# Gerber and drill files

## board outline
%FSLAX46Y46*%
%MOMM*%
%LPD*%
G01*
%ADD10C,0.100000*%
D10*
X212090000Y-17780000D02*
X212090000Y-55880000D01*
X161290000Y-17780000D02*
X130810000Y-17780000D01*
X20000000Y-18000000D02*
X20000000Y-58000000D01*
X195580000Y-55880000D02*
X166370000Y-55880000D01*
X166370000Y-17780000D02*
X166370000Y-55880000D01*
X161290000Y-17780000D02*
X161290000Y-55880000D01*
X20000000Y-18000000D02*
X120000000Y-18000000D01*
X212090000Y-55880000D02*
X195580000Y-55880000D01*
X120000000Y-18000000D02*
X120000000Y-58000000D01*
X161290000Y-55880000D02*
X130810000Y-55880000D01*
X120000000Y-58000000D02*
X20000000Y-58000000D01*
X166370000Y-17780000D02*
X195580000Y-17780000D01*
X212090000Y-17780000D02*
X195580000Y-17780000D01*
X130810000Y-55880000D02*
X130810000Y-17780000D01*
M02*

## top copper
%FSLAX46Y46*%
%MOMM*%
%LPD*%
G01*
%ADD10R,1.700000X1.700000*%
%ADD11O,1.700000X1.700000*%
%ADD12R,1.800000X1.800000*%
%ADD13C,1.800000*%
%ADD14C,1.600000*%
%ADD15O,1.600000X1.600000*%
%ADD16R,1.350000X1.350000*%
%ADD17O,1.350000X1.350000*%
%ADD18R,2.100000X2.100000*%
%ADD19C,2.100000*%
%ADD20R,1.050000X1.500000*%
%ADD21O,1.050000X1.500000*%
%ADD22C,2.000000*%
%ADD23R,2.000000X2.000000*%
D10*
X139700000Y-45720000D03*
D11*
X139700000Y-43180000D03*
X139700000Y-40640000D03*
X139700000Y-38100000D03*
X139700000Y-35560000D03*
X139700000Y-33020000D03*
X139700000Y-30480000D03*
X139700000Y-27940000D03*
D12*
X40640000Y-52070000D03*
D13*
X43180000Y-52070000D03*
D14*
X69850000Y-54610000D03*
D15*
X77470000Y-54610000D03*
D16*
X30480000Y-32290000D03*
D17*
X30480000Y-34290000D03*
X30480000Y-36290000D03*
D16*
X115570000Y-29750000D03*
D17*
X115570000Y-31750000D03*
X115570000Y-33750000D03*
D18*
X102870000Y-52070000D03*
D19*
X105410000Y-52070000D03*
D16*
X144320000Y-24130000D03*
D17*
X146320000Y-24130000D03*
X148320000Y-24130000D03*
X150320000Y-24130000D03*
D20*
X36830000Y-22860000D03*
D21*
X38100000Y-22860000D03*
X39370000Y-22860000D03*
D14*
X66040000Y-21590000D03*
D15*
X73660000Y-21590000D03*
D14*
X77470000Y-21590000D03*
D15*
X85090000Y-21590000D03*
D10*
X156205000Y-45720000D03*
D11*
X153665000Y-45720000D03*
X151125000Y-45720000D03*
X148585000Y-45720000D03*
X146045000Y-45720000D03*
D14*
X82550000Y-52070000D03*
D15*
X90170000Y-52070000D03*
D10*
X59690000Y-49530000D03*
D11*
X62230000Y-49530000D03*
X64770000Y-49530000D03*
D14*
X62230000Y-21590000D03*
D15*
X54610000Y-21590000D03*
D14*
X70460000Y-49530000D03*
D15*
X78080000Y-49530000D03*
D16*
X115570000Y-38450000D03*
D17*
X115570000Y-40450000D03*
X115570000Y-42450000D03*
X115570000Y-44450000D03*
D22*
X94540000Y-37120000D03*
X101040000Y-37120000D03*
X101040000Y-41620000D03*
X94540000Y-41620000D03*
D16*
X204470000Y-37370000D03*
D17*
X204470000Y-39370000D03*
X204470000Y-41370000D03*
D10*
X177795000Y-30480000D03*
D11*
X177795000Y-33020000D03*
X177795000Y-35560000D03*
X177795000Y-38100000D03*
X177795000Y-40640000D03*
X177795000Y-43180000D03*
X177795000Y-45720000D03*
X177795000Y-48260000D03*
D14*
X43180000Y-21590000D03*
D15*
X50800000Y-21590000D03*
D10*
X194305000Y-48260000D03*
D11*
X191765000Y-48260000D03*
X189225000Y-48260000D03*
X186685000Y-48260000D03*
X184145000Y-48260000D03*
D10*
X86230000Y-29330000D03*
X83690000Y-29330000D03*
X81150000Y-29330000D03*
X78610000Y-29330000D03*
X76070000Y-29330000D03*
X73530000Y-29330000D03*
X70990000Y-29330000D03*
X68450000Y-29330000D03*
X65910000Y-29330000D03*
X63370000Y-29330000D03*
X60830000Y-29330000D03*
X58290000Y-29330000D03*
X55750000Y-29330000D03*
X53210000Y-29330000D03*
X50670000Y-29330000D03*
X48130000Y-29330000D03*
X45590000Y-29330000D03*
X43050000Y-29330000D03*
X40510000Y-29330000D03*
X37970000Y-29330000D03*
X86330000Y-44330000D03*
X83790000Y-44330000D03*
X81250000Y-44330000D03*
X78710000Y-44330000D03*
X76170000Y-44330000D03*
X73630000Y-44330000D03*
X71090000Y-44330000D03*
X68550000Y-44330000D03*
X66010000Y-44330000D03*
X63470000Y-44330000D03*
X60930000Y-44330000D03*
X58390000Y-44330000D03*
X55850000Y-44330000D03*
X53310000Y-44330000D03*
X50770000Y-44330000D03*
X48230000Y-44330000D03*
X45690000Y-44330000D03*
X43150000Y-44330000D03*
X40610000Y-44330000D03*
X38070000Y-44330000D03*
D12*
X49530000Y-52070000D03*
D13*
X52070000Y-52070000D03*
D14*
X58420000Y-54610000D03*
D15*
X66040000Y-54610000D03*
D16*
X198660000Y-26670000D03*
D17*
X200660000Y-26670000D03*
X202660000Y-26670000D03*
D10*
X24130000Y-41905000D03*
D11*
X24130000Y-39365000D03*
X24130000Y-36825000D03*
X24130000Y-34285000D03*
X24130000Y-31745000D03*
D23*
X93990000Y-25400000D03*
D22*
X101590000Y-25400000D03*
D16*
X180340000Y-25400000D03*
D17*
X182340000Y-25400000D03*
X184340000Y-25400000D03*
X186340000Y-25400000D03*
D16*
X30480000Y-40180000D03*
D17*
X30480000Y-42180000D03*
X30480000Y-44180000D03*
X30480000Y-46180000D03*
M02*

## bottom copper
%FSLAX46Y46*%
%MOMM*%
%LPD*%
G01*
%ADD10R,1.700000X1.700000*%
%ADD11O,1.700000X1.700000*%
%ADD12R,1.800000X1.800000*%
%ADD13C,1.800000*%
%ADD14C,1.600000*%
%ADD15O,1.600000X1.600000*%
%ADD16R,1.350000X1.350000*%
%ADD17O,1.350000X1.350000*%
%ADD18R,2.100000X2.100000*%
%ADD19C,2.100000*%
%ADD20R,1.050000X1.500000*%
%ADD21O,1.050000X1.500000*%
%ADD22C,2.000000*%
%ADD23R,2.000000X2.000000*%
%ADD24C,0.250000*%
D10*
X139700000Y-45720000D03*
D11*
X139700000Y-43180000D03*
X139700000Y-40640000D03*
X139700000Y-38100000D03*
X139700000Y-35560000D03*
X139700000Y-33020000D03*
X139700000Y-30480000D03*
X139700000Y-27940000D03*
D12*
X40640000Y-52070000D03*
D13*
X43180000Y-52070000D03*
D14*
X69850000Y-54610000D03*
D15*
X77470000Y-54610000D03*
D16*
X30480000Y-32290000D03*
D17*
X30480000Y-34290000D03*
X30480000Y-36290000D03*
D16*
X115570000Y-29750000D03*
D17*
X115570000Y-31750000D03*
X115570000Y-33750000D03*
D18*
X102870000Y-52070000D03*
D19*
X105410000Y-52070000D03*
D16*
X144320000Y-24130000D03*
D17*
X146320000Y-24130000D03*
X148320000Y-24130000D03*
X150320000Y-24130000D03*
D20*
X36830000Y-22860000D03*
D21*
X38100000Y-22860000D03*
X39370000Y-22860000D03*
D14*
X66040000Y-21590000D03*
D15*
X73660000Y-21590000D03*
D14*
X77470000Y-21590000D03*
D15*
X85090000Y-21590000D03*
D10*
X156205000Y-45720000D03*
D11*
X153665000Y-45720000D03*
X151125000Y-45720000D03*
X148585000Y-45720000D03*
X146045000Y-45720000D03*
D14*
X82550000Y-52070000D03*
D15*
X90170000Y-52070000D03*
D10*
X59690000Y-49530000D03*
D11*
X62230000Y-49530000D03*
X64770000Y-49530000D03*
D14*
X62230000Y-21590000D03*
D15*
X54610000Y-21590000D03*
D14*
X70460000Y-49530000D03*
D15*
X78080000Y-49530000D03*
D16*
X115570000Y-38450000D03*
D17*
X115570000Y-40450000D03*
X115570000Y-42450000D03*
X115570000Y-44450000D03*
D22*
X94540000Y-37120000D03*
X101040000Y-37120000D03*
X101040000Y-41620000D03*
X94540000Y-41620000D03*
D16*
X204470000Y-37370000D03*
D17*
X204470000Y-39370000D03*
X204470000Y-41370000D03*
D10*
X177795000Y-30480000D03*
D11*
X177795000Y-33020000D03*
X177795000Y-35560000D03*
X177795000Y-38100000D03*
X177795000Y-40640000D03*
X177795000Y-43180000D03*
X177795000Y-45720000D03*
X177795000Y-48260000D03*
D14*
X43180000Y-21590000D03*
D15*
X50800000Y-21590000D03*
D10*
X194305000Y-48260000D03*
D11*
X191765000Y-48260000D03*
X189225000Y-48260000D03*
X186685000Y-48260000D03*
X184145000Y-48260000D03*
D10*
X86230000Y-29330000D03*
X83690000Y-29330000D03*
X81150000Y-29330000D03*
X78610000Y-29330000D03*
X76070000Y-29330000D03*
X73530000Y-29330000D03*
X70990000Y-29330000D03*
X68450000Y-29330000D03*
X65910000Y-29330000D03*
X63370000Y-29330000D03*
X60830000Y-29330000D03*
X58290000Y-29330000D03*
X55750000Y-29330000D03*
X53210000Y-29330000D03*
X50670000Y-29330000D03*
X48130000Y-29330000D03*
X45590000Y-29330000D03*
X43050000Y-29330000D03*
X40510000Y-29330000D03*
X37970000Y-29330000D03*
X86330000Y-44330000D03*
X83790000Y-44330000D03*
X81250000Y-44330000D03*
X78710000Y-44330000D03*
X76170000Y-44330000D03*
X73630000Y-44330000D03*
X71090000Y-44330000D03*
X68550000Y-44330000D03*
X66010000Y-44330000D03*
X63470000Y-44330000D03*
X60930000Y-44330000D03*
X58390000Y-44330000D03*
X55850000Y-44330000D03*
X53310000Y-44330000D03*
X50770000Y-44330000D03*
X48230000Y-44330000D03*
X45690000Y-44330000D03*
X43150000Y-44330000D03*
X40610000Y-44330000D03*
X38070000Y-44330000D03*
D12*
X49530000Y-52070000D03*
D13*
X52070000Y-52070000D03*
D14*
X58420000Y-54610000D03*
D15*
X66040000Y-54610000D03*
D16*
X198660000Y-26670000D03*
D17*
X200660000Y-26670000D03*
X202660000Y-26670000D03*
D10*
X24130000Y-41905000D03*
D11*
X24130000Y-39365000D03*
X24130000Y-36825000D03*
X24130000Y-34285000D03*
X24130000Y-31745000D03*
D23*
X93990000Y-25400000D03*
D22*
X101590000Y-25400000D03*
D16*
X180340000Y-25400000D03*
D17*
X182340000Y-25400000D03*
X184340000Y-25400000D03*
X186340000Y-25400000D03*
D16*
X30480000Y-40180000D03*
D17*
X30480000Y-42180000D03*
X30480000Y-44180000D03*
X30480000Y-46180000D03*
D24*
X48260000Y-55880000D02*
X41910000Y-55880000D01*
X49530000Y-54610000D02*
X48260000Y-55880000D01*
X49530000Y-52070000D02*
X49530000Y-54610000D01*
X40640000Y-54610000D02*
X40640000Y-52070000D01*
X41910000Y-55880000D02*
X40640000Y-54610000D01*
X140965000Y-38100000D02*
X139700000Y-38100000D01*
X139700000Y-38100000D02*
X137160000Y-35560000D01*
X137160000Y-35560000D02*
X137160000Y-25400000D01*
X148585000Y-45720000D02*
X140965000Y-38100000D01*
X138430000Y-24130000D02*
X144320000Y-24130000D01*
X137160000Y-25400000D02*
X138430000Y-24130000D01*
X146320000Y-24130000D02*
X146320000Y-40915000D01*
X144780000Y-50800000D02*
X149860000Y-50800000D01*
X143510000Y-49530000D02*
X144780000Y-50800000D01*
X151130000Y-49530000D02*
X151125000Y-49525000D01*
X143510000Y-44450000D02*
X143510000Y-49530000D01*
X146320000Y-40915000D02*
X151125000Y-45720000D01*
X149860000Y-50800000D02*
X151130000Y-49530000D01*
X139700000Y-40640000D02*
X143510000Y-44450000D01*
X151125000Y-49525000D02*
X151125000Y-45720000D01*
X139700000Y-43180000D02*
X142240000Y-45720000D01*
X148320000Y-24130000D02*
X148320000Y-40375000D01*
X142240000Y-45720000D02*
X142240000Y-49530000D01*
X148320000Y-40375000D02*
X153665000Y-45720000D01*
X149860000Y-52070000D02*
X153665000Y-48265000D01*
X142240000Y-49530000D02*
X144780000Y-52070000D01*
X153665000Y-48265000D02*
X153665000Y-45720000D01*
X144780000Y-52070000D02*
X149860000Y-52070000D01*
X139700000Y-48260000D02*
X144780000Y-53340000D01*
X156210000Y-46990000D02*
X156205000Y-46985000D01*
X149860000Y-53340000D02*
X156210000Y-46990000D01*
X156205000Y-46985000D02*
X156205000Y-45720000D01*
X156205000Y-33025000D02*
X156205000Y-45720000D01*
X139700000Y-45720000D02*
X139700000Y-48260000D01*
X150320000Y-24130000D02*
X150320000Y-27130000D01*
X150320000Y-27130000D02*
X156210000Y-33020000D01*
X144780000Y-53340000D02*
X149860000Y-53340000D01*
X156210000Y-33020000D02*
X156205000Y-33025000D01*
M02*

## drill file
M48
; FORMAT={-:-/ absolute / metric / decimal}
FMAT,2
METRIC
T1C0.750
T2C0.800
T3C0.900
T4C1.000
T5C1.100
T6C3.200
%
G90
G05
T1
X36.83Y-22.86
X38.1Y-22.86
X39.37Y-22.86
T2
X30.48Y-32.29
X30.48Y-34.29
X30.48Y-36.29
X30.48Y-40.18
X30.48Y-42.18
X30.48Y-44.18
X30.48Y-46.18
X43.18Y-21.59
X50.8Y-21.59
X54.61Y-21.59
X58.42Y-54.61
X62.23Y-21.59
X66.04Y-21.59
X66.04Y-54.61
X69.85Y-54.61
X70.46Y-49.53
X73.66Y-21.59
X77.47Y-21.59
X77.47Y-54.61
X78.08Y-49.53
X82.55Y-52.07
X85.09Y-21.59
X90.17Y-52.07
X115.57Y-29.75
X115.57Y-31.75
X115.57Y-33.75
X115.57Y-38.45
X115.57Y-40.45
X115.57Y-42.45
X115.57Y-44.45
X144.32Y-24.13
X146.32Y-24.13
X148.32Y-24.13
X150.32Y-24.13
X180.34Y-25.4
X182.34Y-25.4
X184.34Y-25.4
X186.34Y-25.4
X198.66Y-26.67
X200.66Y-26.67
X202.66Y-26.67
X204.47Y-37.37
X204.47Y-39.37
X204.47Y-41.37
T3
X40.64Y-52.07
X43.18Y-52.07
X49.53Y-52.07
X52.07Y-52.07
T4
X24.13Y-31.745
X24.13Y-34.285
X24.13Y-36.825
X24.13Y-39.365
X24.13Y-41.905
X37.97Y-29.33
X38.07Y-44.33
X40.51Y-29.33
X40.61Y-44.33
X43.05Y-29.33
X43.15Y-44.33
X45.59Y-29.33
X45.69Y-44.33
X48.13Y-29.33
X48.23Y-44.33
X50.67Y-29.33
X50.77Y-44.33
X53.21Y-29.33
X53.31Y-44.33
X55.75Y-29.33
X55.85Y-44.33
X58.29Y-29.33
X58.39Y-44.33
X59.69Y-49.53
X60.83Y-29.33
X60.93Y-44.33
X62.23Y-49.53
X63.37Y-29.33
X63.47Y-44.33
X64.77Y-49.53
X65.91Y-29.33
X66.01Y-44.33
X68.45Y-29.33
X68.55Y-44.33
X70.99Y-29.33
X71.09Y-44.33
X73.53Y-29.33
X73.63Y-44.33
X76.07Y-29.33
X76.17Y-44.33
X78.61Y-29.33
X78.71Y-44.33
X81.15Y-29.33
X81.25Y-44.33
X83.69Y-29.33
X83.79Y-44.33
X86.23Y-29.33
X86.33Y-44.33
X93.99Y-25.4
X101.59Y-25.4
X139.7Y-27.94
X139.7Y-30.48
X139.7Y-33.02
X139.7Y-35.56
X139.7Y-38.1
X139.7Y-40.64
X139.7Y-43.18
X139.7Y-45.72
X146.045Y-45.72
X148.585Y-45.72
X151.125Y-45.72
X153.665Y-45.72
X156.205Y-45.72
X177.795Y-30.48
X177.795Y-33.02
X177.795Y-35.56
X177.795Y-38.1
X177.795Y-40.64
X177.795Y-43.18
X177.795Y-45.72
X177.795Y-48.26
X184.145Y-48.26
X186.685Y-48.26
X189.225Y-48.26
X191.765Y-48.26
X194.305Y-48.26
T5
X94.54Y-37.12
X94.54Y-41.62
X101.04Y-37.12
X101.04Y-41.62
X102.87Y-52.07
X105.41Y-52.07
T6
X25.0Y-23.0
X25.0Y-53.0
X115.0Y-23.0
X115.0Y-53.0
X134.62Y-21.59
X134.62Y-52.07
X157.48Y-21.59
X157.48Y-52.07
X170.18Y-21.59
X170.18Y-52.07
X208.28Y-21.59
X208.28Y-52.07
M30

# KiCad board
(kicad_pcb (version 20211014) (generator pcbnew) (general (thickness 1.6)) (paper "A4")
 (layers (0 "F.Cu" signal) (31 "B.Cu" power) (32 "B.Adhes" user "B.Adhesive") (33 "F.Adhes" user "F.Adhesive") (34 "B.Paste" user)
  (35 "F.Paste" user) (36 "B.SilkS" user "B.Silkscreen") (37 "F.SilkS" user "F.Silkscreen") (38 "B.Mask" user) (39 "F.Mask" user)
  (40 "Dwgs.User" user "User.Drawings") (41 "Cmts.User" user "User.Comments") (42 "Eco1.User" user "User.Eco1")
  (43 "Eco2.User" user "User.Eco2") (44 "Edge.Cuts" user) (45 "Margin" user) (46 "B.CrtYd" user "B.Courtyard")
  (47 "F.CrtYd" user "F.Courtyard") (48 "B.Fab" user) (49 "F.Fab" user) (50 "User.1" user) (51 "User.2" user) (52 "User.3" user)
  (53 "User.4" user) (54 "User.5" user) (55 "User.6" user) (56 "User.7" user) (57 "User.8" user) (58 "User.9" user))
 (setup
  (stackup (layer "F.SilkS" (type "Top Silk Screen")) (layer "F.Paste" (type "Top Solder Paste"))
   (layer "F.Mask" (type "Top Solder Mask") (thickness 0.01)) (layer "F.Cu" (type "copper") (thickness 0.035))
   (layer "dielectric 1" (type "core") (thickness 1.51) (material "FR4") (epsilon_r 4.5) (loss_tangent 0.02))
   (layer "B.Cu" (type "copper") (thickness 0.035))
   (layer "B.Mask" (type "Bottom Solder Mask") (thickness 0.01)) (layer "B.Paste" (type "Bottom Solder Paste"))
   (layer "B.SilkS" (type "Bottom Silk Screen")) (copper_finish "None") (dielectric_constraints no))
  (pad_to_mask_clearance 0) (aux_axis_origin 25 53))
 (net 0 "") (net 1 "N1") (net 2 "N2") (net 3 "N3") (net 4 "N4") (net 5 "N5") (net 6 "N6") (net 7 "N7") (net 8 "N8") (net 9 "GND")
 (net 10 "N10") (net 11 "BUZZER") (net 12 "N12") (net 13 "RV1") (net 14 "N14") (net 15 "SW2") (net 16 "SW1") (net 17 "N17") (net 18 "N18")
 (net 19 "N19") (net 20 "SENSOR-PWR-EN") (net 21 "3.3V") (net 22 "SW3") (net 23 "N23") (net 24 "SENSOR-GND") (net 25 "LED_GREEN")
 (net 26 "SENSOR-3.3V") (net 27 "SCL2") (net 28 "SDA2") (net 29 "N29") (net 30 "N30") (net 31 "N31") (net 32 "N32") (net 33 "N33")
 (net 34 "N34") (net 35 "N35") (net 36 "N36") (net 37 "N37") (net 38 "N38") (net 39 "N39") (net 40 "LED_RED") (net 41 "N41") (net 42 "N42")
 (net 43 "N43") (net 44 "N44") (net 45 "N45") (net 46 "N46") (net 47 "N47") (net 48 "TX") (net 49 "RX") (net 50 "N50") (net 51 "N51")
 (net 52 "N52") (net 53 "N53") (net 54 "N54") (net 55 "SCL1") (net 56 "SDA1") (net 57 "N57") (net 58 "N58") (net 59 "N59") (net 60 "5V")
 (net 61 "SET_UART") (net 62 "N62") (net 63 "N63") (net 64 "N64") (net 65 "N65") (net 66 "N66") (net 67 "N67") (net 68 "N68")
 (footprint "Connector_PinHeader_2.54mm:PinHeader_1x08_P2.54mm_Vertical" (layer "F.Cu") (at 139.7 45.72 180)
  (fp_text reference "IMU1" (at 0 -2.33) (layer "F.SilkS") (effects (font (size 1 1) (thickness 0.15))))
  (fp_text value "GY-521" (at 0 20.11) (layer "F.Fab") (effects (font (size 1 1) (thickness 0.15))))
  (pad "1" thru_hole rect (at 0 0 180) (size 1.7 1.7) (drill 1) (layers *.Cu *.Mask) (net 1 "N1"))
  (pad "2" thru_hole oval (at 0 2.54 180) (size 1.7 1.7) (drill 1) (layers *.Cu *.Mask) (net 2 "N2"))
  (pad "3" thru_hole oval (at 0 5.08 180) (size 1.7 1.7) (drill 1) (layers *.Cu *.Mask) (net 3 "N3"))
  (pad "4" thru_hole oval (at 0 7.62 180) (size 1.7 1.7) (drill 1) (layers *.Cu *.Mask) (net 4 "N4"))
  (pad "5" thru_hole oval (at 0 10.16 180) (size 1.7 1.7) (drill 1) (layers *.Cu *.Mask) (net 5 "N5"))
  (pad "6" thru_hole oval (at 0 12.7 180) (size 1.7 1.7) (drill 1) (layers *.Cu *.Mask) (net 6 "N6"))
  (pad "7" thru_hole oval (at 0 15.24 180) (size 1.7 1.7) (drill 1) (layers *.Cu *.Mask) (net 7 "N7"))
  (pad "8" thru_hole oval (at 0 17.78 180) (size 1.7 1.7) (drill 1) (layers *.Cu *.Mask) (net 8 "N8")))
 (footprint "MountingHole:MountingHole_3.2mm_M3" (layer "F.Cu") (at 157.48 21.59)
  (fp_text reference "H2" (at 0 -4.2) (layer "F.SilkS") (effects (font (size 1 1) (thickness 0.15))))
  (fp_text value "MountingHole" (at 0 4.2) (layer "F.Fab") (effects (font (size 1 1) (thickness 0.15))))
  (pad "" np_thru_hole circle (at 0 0) (size 3.2 3.2) (drill 3.2) (layers *.Cu *.Mask)))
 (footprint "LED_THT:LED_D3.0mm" (layer "F.Cu") (at 40.64 52.07)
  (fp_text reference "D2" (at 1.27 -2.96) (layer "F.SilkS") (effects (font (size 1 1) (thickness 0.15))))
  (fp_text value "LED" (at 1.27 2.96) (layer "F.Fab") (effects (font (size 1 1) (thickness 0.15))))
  (pad "1" thru_hole rect (at 0 0) (size 1.8 1.8) (drill 0.9) (layers *.Cu *.Mask) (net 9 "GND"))
  (pad "2" thru_hole circle (at 2.54 0) (size 1.8 1.8) (drill 0.9) (layers *.Cu *.Mask) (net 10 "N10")))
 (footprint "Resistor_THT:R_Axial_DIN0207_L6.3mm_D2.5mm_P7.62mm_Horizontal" (layer "F.Cu") (at 69.85 54.61)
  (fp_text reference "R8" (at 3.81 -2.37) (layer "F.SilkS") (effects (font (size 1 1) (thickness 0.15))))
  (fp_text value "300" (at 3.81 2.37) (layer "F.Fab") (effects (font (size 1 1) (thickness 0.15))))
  (pad "1" thru_hole circle (at 0 0) (size 1.6 1.6) (drill 0.8) (layers *.Cu *.Mask) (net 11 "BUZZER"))
  (pad "2" thru_hole oval (at 7.62 0) (size 1.6 1.6) (drill 0.8) (layers *.Cu *.Mask) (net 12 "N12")))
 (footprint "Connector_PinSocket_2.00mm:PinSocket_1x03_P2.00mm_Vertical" (layer "F.Cu") (at 30.48 32.29)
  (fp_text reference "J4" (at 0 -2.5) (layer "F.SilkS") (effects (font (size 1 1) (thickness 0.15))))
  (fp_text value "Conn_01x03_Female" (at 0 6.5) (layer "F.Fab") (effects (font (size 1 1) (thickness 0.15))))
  (pad "1" thru_hole rect (at 0 0) (size 1.35 1.35) (drill 0.8) (layers *.Cu *.Mask) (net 9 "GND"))
  (pad "2" thru_hole oval (at 0 2) (size 1.35 1.35) (drill 0.8) (layers *.Cu *.Mask) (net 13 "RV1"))
  (pad "3" thru_hole oval (at 0 4) (size 1.35 1.35) (drill 0.8) (layers *.Cu *.Mask) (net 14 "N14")))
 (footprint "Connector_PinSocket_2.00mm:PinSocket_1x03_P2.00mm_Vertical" (layer "F.Cu") (at 115.57 29.75)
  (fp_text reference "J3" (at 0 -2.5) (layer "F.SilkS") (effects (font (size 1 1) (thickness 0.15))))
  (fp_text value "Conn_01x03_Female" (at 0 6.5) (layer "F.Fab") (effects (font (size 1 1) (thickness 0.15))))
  (pad "1" thru_hole rect (at 0 0) (size 1.35 1.35) (drill 0.8) (layers *.Cu *.Mask) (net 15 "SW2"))
  (pad "2" thru_hole oval (at 0 2) (size 1.35 1.35) (drill 0.8) (layers *.Cu *.Mask) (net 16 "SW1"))
  (pad "3" thru_hole oval (at 0 4) (size 1.35 1.35) (drill 0.8) (layers *.Cu *.Mask) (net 9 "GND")))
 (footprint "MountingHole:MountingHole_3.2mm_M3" (layer "F.Cu") (at 208.28 21.59)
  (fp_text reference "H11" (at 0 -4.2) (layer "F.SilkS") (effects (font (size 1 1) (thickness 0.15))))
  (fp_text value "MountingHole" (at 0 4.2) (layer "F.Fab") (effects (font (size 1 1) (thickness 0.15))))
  (pad "" np_thru_hole circle (at 0 0) (size 3.2 3.2) (drill 3.2) (layers *.Cu *.Mask)))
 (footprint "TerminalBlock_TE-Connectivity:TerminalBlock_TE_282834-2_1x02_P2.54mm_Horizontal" (layer "F.Cu") (at 102.87 52.07)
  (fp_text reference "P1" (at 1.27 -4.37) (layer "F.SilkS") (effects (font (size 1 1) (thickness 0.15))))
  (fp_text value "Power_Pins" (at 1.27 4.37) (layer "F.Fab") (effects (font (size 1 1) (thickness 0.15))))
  (pad "1" thru_hole rect (at 0 0) (size 2.1 2.1) (drill 1.1) (layers *.Cu *.Mask) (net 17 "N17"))
  (pad "2" thru_hole circle (at 2.54 0) (size 2.1 2.1) (drill 1.1) (layers *.Cu *.Mask) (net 9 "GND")))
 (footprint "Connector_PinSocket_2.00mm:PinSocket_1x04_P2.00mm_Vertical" (layer "F.Cu") (at 144.32 24.13 90)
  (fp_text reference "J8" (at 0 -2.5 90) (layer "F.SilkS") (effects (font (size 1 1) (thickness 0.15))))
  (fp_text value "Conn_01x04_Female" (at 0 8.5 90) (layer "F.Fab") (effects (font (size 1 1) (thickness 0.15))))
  (pad "1" thru_hole rect (at 0 0 90) (size 1.35 1.35) (drill 0.8) (layers *.Cu *.Mask) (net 4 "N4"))
  (pad "2" thru_hole oval (at 0 2 90) (size 1.35 1.35) (drill 0.8) (layers *.Cu *.Mask) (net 3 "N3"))
  (pad "3" thru_hole oval (at 0 4 90) (size 1.35 1.35) (drill 0.8) (layers *.Cu *.Mask) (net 2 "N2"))
  (pad "4" thru_hole oval (at 0 6 90) (size 1.35 1.35) (drill 0.8) (layers *.Cu *.Mask) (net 1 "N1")))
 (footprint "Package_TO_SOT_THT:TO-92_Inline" (layer "F.Cu") (at 36.83 22.86)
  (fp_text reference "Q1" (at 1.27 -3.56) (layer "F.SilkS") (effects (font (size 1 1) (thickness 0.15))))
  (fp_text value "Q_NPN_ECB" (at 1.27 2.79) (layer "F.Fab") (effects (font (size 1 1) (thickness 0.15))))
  (pad "1" thru_hole rect (at 0 0) (size 1.05 1.5) (drill 0.75) (layers *.Cu *.Mask) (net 9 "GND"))
  (pad "2" thru_hole oval (at 1.27 0) (size 1.05 1.5) (drill 0.75) (layers *.Cu *.Mask) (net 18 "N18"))
  (pad "3" thru_hole oval (at 2.54 0) (size 1.05 1.5) (drill 0.75) (layers *.Cu *.Mask) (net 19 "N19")))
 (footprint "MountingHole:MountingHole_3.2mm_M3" (layer "F.Cu") (at 115 23)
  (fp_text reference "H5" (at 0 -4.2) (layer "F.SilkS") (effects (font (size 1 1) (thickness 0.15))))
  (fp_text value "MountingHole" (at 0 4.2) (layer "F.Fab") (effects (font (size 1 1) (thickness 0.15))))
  (pad "" np_thru_hole circle (at 0 0) (size 3.2 3.2) (drill 3.2) (layers *.Cu *.Mask)))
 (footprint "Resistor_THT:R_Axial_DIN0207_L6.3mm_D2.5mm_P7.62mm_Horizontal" (layer "F.Cu") (at 66.04 21.59)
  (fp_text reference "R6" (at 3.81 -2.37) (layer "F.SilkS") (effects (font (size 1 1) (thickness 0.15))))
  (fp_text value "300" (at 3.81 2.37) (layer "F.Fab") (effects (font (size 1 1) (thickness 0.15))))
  (pad "1" thru_hole circle (at 0 0) (size 1.6 1.6) (drill 0.8) (layers *.Cu *.Mask) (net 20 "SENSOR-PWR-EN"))
  (pad "2" thru_hole oval (at 7.62 0) (size 1.6 1.6) (drill 0.8) (layers *.Cu *.Mask) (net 19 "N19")))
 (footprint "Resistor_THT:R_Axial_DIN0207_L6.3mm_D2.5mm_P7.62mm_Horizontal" (layer "F.Cu") (at 77.47 21.59)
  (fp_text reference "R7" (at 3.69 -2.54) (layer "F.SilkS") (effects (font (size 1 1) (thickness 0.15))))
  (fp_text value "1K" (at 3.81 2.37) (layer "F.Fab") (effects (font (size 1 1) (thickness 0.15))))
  (pad "1" thru_hole circle (at 0 0) (size 1.6 1.6) (drill 0.8) (layers *.Cu *.Mask) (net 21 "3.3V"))
  (pad "2" thru_hole oval (at 7.62 0) (size 1.6 1.6) (drill 0.8) (layers *.Cu *.Mask) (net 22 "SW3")))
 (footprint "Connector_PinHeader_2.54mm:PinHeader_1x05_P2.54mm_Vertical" (layer "F.Cu") (at 156.205 45.72 -90)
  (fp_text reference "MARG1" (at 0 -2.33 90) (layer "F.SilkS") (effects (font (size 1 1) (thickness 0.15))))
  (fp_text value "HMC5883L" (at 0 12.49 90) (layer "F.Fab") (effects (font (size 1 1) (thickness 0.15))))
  (pad "1" thru_hole rect (at 0 0 270) (size 1.7 1.7) (drill 1) (layers *.Cu *.Mask) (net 1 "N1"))
  (pad "2" thru_hole oval (at 0 2.54 270) (size 1.7 1.7) (drill 1) (layers *.Cu *.Mask) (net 2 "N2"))
  (pad "3" thru_hole oval (at 0 5.08 270) (size 1.7 1.7) (drill 1) (layers *.Cu *.Mask) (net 3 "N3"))
  (pad "4" thru_hole oval (at 0 7.62 270) (size 1.7 1.7) (drill 1) (layers *.Cu *.Mask) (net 4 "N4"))
  (pad "5" thru_hole oval (at 0 10.16 270) (size 1.7 1.7) (drill 1) (layers *.Cu *.Mask) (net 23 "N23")))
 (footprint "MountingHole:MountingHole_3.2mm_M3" (layer "F.Cu") (at 25 53)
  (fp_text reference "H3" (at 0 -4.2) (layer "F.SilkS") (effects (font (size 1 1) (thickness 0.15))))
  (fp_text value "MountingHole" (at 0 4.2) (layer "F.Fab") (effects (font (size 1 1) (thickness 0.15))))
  (pad "" np_thru_hole circle (at 0 0) (size 3.2 3.2) (drill 3.2) (layers *.Cu *.Mask)))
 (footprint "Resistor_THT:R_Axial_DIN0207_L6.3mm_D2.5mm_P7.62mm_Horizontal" (layer "F.Cu") (at 82.55 52.07)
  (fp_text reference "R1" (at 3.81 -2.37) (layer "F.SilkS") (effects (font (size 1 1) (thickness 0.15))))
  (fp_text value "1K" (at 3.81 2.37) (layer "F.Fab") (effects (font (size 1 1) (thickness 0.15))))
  (pad "1" thru_hole circle (at 0 0) (size 1.6 1.6) (drill 0.8) (layers *.Cu *.Mask) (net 21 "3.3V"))
  (pad "2" thru_hole oval (at 7.62 0) (size 1.6 1.6) (drill 0.8) (layers *.Cu *.Mask) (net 16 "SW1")))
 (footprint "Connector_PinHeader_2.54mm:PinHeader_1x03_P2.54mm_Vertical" (layer "F.Cu") (at 59.69 49.53 90)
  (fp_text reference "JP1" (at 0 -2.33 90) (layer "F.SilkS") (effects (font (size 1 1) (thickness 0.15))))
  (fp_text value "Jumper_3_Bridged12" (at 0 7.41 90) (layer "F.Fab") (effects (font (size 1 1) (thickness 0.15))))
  (pad "1" thru_hole rect (at 0 0 90) (size 1.7 1.7) (drill 1) (layers *.Cu *.Mask) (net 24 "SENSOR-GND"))
  (pad "2" thru_hole oval (at 0 2.54 90) (size 1.7 1.7) (drill 1) (layers *.Cu *.Mask) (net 9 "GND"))
  (pad "3" thru_hole oval (at 0 5.08 90) (size 1.7 1.7) (drill 1) (layers *.Cu *.Mask) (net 18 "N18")))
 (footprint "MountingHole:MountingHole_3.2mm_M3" (layer "F.Cu") (at 170.18 21.59)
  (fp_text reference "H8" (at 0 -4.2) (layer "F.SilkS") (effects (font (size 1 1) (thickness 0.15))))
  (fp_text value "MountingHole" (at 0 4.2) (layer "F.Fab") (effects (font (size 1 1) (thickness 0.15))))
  (pad "" np_thru_hole circle (at 0 0) (size 3.2 3.2) (drill 3.2) (layers *.Cu *.Mask)))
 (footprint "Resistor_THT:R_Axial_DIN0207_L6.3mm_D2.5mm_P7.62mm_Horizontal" (layer "F.Cu") (at 62.23 21.59 180)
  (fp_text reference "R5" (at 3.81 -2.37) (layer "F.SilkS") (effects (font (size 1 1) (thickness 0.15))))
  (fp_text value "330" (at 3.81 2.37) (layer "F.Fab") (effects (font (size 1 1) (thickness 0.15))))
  (pad "1" thru_hole circle (at 0 0 180) (size 1.6 1.6) (drill 0.8) (layers *.Cu *.Mask) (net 21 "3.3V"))
  (pad "2" thru_hole oval (at 7.62 0 180) (size 1.6 1.6) (drill 0.8) (layers *.Cu *.Mask) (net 14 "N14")))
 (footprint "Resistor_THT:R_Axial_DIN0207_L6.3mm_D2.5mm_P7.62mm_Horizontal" (layer "F.Cu") (at 70.46 49.53)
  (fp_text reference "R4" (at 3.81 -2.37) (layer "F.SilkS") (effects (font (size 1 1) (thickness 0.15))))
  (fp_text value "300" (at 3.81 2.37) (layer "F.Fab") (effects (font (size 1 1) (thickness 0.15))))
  (pad "1" thru_hole circle (at 0 0) (size 1.6 1.6) (drill 0.8) (layers *.Cu *.Mask) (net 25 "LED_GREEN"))
  (pad "2" thru_hole oval (at 7.62 0) (size 1.6 1.6) (drill 0.8) (layers *.Cu *.Mask) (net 10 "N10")))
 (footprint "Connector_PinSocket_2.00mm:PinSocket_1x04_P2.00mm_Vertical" (layer "F.Cu") (at 115.57 38.45)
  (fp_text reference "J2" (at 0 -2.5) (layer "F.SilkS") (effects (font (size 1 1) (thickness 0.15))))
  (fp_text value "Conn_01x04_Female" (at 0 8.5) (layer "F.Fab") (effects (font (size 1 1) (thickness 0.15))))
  (pad "1" thru_hole rect (at 0 0) (size 1.35 1.35) (drill 0.8) (layers *.Cu *.Mask) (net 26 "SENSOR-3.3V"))
  (pad "2" thru_hole oval (at 0 2) (size 1.35 1.35) (drill 0.8) (layers *.Cu *.Mask) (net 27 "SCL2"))
  (pad "3" thru_hole oval (at 0 4) (size 1.35 1.35) (drill 0.8) (layers *.Cu *.Mask) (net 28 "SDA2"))
  (pad "4" thru_hole oval (at 0 6) (size 1.35 1.35) (drill 0.8) (layers *.Cu *.Mask) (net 24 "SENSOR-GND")))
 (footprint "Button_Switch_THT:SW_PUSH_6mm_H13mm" (layer "F.Cu") (at 94.54 37.12)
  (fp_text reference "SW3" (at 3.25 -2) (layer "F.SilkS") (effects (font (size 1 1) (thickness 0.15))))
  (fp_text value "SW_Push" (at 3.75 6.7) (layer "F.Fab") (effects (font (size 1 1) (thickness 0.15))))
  (pad "1" thru_hole circle (at 0 0 90) (size 2 2) (drill 1.1) (layers *.Cu *.Mask) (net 9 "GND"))
  (pad "1" thru_hole circle (at 6.5 0 90) (size 2 2) (drill 1.1) (layers *.Cu *.Mask) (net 9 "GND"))
  (pad "2" thru_hole circle (at 6.5 4.5 90) (size 2 2) (drill 1.1) (layers *.Cu *.Mask) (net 22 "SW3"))
  (pad "2" thru_hole circle (at 0 4.5 90) (size 2 2) (drill 1.1) (layers *.Cu *.Mask) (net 22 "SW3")))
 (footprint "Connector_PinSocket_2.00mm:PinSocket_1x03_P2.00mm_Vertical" (layer "F.Cu") (at 204.47 37.37)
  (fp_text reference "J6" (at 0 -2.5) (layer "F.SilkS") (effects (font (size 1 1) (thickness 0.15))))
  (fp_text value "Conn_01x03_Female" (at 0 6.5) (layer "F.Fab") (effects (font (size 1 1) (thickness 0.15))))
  (pad "1" thru_hole rect (at 0 0) (size 1.35 1.35) (drill 0.8) (layers *.Cu *.Mask) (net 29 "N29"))
  (pad "2" thru_hole oval (at 0 2) (size 1.35 1.35) (drill 0.8) (layers *.Cu *.Mask) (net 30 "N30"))
  (pad "3" thru_hole oval (at 0 4) (size 1.35 1.35) (drill 0.8) (layers *.Cu *.Mask) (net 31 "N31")))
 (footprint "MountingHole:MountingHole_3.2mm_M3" (layer "F.Cu") (at 134.62 21.59)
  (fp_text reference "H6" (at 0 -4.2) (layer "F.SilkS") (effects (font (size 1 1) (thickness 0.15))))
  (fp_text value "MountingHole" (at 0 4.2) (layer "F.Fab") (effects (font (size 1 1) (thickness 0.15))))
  (pad "" np_thru_hole circle (at 0 0) (size 3.2 3.2) (drill 3.2) (layers *.Cu *.Mask)))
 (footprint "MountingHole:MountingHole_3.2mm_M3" (layer "F.Cu") (at 170.18 52.07)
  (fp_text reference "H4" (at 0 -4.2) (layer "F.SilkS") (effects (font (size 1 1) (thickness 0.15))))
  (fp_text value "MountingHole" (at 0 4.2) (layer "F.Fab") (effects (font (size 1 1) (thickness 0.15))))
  (pad "" np_thru_hole circle (at 0 0) (size 3.2 3.2) (drill 3.2) (layers *.Cu *.Mask)))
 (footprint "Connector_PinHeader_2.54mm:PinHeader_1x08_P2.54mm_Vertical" (layer "F.Cu") (at 177.795 30.48)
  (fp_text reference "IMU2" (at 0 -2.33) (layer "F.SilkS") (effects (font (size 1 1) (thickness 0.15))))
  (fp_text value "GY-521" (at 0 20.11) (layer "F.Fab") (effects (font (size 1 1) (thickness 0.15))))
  (pad "1" thru_hole rect (at 0 0) (size 1.7 1.7) (drill 1) (layers *.Cu *.Mask) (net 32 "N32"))
  (pad "2" thru_hole oval (at 0 2.54) (size 1.7 1.7) (drill 1) (layers *.Cu *.Mask) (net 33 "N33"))
  (pad "3" thru_hole oval (at 0 5.08) (size 1.7 1.7) (drill 1) (layers *.Cu *.Mask) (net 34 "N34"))
  (pad "4" thru_hole oval (at 0 7.62) (size 1.7 1.7) (drill 1) (layers *.Cu *.Mask) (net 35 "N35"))
  (pad "5" thru_hole oval (at 0 10.16) (size 1.7 1.7) (drill 1) (layers *.Cu *.Mask) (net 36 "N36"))
  (pad "6" thru_hole oval (at 0 12.7) (size 1.7 1.7) (drill 1) (layers *.Cu *.Mask) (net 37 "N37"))
  (pad "7" thru_hole oval (at 0 15.24) (size 1.7 1.7) (drill 1) (layers *.Cu *.Mask) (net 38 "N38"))
  (pad "8" thru_hole oval (at 0 17.78) (size 1.7 1.7) (drill 1) (layers *.Cu *.Mask) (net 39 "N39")))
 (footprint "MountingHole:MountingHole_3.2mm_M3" (layer "F.Cu") (at 208.28 52.07)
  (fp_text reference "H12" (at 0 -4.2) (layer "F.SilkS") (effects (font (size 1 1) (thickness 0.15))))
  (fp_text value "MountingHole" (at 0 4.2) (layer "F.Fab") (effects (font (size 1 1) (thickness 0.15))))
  (pad "" np_thru_hole circle (at 0 0) (size 3.2 3.2) (drill 3.2) (layers *.Cu *.Mask)))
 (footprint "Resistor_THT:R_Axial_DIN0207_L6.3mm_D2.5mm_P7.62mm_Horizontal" (layer "F.Cu") (at 43.18 21.59)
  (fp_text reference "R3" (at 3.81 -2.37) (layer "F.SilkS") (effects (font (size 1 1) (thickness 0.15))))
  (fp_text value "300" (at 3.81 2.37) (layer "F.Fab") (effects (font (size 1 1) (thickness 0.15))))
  (pad "1" thru_hole circle (at 0 0) (size 1.6 1.6) (drill 0.8) (layers *.Cu *.Mask) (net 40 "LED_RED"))
  (pad "2" thru_hole oval (at 7.62 0) (size 1.6 1.6) (drill 0.8) (layers *.Cu *.Mask) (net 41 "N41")))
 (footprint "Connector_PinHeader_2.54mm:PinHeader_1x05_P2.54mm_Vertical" (layer "F.Cu") (at 194.305 48.26 -90)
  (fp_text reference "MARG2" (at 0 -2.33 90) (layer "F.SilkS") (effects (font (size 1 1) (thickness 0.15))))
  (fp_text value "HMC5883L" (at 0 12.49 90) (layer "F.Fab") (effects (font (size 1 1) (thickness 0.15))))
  (pad "1" thru_hole rect (at 0 0 270) (size 1.7 1.7) (drill 1) (layers *.Cu *.Mask) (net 32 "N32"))
  (pad "2" thru_hole oval (at 0 2.54 270) (size 1.7 1.7) (drill 1) (layers *.Cu *.Mask) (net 33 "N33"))
  (pad "3" thru_hole oval (at 0 5.08 270) (size 1.7 1.7) (drill 1) (layers *.Cu *.Mask) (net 34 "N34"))
  (pad "4" thru_hole oval (at 0 7.62 270) (size 1.7 1.7) (drill 1) (layers *.Cu *.Mask) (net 35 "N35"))
  (pad "5" thru_hole oval (at 0 10.16 270) (size 1.7 1.7) (drill 1) (layers *.Cu *.Mask) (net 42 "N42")))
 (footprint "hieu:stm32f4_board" (layer "F.Cu") (at 86.23 29.33 -90)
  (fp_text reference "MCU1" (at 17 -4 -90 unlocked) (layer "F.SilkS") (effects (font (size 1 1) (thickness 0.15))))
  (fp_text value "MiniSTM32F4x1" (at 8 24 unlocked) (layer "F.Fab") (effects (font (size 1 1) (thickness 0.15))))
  (pad "1" thru_hole rect (at 0 0 270) (size 1.7 1.7) (drill 1) (layers *.Cu *.Mask) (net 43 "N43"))
  (pad "2" thru_hole rect (at 0 2.54 270) (size 1.7 1.7) (drill 1) (layers *.Cu *.Mask) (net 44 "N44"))
  (pad "3" thru_hole rect (at 0 5.08 270) (size 1.7 1.7) (drill 1) (layers *.Cu *.Mask) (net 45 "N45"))
  (pad "4" thru_hole rect (at 0 7.62 270) (size 1.7 1.7) (drill 1) (layers *.Cu *.Mask) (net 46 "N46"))
  (pad "5" thru_hole rect (at 0 10.16 270) (size 1.7 1.7) (drill 1) (layers *.Cu *.Mask) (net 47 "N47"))
  (pad "6" thru_hole rect (at 0 12.7 270) (size 1.7 1.7) (drill 1) (layers *.Cu *.Mask) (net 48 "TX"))
  (pad "7" thru_hole rect (at 0 15.24 270) (size 1.7 1.7) (drill 1) (layers *.Cu *.Mask) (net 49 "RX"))
  (pad "8" thru_hole rect (at 0 17.78 270) (size 1.7 1.7) (drill 1) (layers *.Cu *.Mask) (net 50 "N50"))
  (pad "9" thru_hole rect (at 0 20.32 270) (size 1.7 1.7) (drill 1) (layers *.Cu *.Mask) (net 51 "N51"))
  (pad "10" thru_hole rect (at 0 22.86 270) (size 1.7 1.7) (drill 1) (layers *.Cu *.Mask) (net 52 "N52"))
  (pad "11" thru_hole rect (at 0 25.4 270) (size 1.7 1.7) (drill 1) (layers *.Cu *.Mask) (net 28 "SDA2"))
  (pad "12" thru_hole rect (at 0 27.94 270) (size 1.7 1.7) (drill 1) (layers *.Cu *.Mask) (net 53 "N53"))
  (pad "13" thru_hole rect (at 0 30.48 270) (size 1.7 1.7) (drill 1) (layers *.Cu *.Mask) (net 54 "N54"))
  (pad "14" thru_hole rect (at 0 33.02 270) (size 1.7 1.7) (drill 1) (layers *.Cu *.Mask) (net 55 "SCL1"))
  (pad "15" thru_hole rect (at 0 35.56 270) (size 1.7 1.7) (drill 1) (layers *.Cu *.Mask) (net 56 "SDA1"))
  (pad "16" thru_hole rect (at 0 38.1 270) (size 1.7 1.7) (drill 1) (layers *.Cu *.Mask) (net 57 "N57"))
  (pad "17" thru_hole rect (at 0 40.64 270) (size 1.7 1.7) (drill 1) (layers *.Cu *.Mask) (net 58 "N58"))
  (pad "18" thru_hole rect (at 0 43.18 270) (size 1.7 1.7) (drill 1) (layers *.Cu *.Mask) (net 21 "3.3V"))
  (pad "19" thru_hole rect (at 0 45.72 270) (size 1.7 1.7) (drill 1) (layers *.Cu *.Mask) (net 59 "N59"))
  (pad "20" thru_hole rect (at 0 48.26 270) (size 1.7 1.7) (drill 1) (layers *.Cu *.Mask) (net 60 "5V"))
  (pad "21" thru_hole rect (at 15 -0.1 270) (size 1.7 1.7) (drill 1) (layers *.Cu *.Mask) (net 17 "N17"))
  (pad "22" thru_hole rect (at 15 2.44 270) (size 1.7 1.7) (drill 1) (layers *.Cu *.Mask) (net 9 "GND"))
  (pad "23" thru_hole rect (at 15 4.98 270) (size 1.7 1.7) (drill 1) (layers *.Cu *.Mask) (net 26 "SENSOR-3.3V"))
  (pad "24" thru_hole rect (at 15 7.52 270) (size 1.7 1.7) (drill 1) (layers *.Cu *.Mask) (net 27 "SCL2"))
  (pad "25" thru_hole rect (at 15 10.06 270) (size 1.7 1.7) (drill 1) (layers *.Cu *.Mask) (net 20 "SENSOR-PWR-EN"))
  (pad "26" thru_hole rect (at 15 12.6 270) (size 1.7 1.7) (drill 1) (layers *.Cu *.Mask) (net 25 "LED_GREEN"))
  (pad "27" thru_hole rect (at 15 15.14 270) (size 1.7 1.7) (drill 1) (layers *.Cu *.Mask) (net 40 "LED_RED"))
  (pad "28" thru_hole rect (at 15 17.68 270) (size 1.7 1.7) (drill 1) (layers *.Cu *.Mask) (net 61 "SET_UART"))
  (pad "29" thru_hole rect (at 15 20.22 270) (size 1.7 1.7) (drill 1) (layers *.Cu *.Mask) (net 11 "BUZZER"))
  (pad "30" thru_hole rect (at 15 22.76 270) (size 1.7 1.7) (drill 1) (layers *.Cu *.Mask) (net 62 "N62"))
  (pad "31" thru_hole rect (at 15 25.3 270) (size 1.7 1.7) (drill 1) (layers *.Cu *.Mask) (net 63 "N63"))
  (pad "32" thru_hole rect (at 15 27.84 270) (size 1.7 1.7) (drill 1) (layers *.Cu *.Mask) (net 22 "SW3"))
  (pad "33" thru_hole rect (at 15 30.38 270) (size 1.7 1.7) (drill 1) (layers *.Cu *.Mask) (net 15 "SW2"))
  (pad "34" thru_hole rect (at 15 32.92 270) (size 1.7 1.7) (drill 1) (layers *.Cu *.Mask) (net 16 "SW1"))
  (pad "35" thru_hole rect (at 15 35.46 270) (size 1.7 1.7) (drill 1) (layers *.Cu *.Mask) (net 13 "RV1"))
  (pad "36" thru_hole rect (at 15 38 270) (size 1.7 1.7) (drill 1) (layers *.Cu *.Mask) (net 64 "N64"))
  (pad "37" thru_hole rect (at 15 40.54 270) (size 1.7 1.7) (drill 1) (layers *.Cu *.Mask) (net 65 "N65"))
  (pad "38" thru_hole rect (at 15 43.08 270) (size 1.7 1.7) (drill 1) (layers *.Cu *.Mask) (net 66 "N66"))
  (pad "39" thru_hole rect (at 15 45.62 270) (size 1.7 1.7) (drill 1) (layers *.Cu *.Mask) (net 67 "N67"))
  (pad "40" thru_hole rect (at 15 48.16 270) (size 1.7 1.7) (drill 1) (layers *.Cu *.Mask) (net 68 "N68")))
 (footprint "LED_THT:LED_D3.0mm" (layer "F.Cu") (at 49.53 52.07)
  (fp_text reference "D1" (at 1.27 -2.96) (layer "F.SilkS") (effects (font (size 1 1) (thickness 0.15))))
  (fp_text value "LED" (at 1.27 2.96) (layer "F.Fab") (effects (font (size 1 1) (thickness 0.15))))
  (pad "1" thru_hole rect (at 0 0) (size 1.8 1.8) (drill 0.9) (layers *.Cu *.Mask) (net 9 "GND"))
  (pad "2" thru_hole circle (at 2.54 0) (size 1.8 1.8) (drill 0.9) (layers *.Cu *.Mask) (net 41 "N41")))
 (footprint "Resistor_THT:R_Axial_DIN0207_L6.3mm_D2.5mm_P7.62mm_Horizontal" (layer "F.Cu") (at 58.42 54.61)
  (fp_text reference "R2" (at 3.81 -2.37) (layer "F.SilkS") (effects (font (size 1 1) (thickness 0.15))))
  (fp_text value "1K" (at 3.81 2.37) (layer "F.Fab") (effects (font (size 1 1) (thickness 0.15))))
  (pad "1" thru_hole circle (at 0 0) (size 1.6 1.6) (drill 0.8) (layers *.Cu *.Mask) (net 21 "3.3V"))
  (pad "2" thru_hole oval (at 7.62 0) (size 1.6 1.6) (drill 0.8) (layers *.Cu *.Mask) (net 15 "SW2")))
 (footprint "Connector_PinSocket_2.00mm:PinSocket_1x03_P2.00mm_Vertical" (layer "F.Cu") (at 198.66 26.67 90)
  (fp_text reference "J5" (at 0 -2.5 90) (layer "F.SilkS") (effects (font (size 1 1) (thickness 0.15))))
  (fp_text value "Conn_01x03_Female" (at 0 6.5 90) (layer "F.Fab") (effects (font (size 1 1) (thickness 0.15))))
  (pad "1" thru_hole rect (at 0 0 90) (size 1.35 1.35) (drill 0.8) (layers *.Cu *.Mask) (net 29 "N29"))
  (pad "2" thru_hole oval (at 0 2 90) (size 1.35 1.35) (drill 0.8) (layers *.Cu *.Mask) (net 30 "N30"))
  (pad "3" thru_hole oval (at 0 4 90) (size 1.35 1.35) (drill 0.8) (layers *.Cu *.Mask) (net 31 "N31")))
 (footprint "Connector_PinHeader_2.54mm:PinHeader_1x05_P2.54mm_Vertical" (layer "F.Cu") (at 24.13 41.905 180)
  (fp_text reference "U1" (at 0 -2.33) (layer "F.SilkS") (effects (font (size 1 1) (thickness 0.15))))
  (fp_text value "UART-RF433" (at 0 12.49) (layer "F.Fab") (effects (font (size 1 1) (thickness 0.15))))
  (pad "1" thru_hole rect (at 0 0 180) (size 1.7 1.7) (drill 1) (layers *.Cu *.Mask) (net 60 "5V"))
  (pad "2" thru_hole oval (at 0 2.54 180) (size 1.7 1.7) (drill 1) (layers *.Cu *.Mask) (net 9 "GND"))
  (pad "3" thru_hole oval (at 0 5.08 180) (size 1.7 1.7) (drill 1) (layers *.Cu *.Mask) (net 48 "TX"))
  (pad "4" thru_hole oval (at 0 7.62 180) (size 1.7 1.7) (drill 1) (layers *.Cu *.Mask) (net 49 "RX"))
  (pad "5" thru_hole oval (at 0 10.16 180) (size 1.7 1.7) (drill 1) (layers *.Cu *.Mask) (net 61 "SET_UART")))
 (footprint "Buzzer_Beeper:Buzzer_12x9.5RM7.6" (layer "F.Cu") (at 93.99 25.4)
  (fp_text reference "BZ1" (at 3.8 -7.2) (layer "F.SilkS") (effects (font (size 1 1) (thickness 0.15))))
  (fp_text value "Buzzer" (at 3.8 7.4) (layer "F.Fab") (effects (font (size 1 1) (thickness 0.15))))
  (pad "1" thru_hole rect (at 0 0) (size 2 2) (drill 1) (layers *.Cu *.Mask) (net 12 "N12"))
  (pad "2" thru_hole circle (at 7.6 0) (size 2 2) (drill 1) (layers *.Cu *.Mask) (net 9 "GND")))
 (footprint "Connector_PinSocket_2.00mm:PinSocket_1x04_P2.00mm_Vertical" (layer "F.Cu") (at 180.34 25.4 90)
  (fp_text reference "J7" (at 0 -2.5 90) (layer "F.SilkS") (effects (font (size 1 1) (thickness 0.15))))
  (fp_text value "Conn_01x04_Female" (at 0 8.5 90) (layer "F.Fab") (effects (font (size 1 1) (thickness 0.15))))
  (pad "1" thru_hole rect (at 0 0 90) (size 1.35 1.35) (drill 0.8) (layers *.Cu *.Mask) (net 35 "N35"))
  (pad "2" thru_hole oval (at 0 2 90) (size 1.35 1.35) (drill 0.8) (layers *.Cu *.Mask) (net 34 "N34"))
  (pad "3" thru_hole oval (at 0 4 90) (size 1.35 1.35) (drill 0.8) (layers *.Cu *.Mask) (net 33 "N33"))
  (pad "4" thru_hole oval (at 0 6 90) (size 1.35 1.35) (drill 0.8) (layers *.Cu *.Mask) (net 32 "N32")))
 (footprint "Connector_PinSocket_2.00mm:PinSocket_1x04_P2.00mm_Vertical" (layer "F.Cu") (at 30.48 40.18)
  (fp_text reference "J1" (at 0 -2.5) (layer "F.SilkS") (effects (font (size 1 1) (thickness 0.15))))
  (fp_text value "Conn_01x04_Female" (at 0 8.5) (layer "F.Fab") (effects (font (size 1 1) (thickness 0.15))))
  (pad "1" thru_hole rect (at 0 0) (size 1.35 1.35) (drill 0.8) (layers *.Cu *.Mask) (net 26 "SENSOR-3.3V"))
  (pad "2" thru_hole oval (at 0 2) (size 1.35 1.35) (drill 0.8) (layers *.Cu *.Mask) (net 55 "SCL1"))
  (pad "3" thru_hole oval (at 0 4) (size 1.35 1.35) (drill 0.8) (layers *.Cu *.Mask) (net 56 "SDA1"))
  (pad "4" thru_hole oval (at 0 6) (size 1.35 1.35) (drill 0.8) (layers *.Cu *.Mask) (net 24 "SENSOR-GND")))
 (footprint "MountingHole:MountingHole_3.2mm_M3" (layer "F.Cu") (at 157.48 52.07)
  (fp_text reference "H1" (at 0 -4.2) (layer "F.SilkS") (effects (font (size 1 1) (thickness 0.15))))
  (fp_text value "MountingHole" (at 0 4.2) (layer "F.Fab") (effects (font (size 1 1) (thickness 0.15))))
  (pad "" np_thru_hole circle (at 0 0) (size 3.2 3.2) (drill 3.2) (layers *.Cu *.Mask)))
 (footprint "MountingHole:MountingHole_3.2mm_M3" (layer "F.Cu") (at 25 23)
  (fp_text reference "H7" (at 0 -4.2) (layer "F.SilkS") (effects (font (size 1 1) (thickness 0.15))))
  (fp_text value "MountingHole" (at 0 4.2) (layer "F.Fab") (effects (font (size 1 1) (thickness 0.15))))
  (pad "" np_thru_hole circle (at 0 0) (size 3.2 3.2) (drill 3.2) (layers *.Cu *.Mask)))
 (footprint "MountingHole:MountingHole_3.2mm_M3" (layer "F.Cu") (at 115 53)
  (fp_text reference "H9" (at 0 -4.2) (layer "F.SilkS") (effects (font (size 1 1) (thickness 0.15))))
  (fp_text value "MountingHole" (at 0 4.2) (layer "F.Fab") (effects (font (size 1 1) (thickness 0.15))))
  (pad "" np_thru_hole circle (at 0 0) (size 3.2 3.2) (drill 3.2) (layers *.Cu *.Mask)))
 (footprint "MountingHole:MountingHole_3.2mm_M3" (layer "F.Cu") (at 134.62 52.07)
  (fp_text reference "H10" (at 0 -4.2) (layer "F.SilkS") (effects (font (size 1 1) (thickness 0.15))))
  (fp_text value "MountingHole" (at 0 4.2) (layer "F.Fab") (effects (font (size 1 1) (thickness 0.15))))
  (pad "" np_thru_hole circle (at 0 0) (size 3.2 3.2) (drill 3.2) (layers *.Cu *.Mask)))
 (gr_line (start 212.09 17.78) (end 212.09 55.88) (layer "Edge.Cuts") (width 0.1))
 (gr_line (start 161.29 17.78) (end 130.81 17.78) (layer "Edge.Cuts") (width 0.1))
 (gr_line (start 20 18) (end 20 58) (layer "Edge.Cuts") (width 0.1))
 (gr_line (start 195.58 55.88) (end 166.37 55.88) (layer "Edge.Cuts") (width 0.1))
 (gr_line (start 166.37 17.78) (end 166.37 55.88) (layer "Edge.Cuts") (width 0.1))
 (gr_line (start 161.29 17.78) (end 161.29 55.88) (layer "Edge.Cuts") (width 0.1))
 (gr_line (start 20 18) (end 120 18) (layer "Edge.Cuts") (width 0.1))
 (gr_line (start 212.09 55.88) (end 195.58 55.88) (layer "Edge.Cuts") (width 0.1))
 (gr_line (start 120 18) (end 120 58) (layer "Edge.Cuts") (width 0.1))
 (gr_line (start 161.29 55.88) (end 130.81 55.88) (layer "Edge.Cuts") (width 0.1))
 (gr_line (start 120 58) (end 20 58) (layer "Edge.Cuts") (width 0.1))
 (gr_line (start 166.37 17.78) (end 195.58 17.78) (layer "Edge.Cuts") (width 0.1))
 (gr_line (start 212.09 17.78) (end 195.58 17.78) (layer "Edge.Cuts") (width 0.1))
 (gr_line (start 130.81 55.88) (end 130.81 17.78) (layer "Edge.Cuts") (width 0.1))
 (segment (start 48.26 55.88) (end 41.91 55.88) (width 0.25) (layer "B.Cu") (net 9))
 (segment (start 49.53 54.61) (end 48.26 55.88) (width 0.25) (layer "B.Cu") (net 9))
 (segment (start 49.53 52.07) (end 49.53 54.61) (width 0.25) (layer "B.Cu") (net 9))
 (segment (start 40.64 54.61) (end 40.64 52.07) (width 0.25) (layer "B.Cu") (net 9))
 (segment (start 41.91 55.88) (end 40.64 54.61) (width 0.25) (layer "B.Cu") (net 9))
 (segment (start 140.965 38.1) (end 139.7 38.1) (width 0.25) (layer "B.Cu") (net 4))
 (segment (start 139.7 38.1) (end 137.16 35.56) (width 0.25) (layer "B.Cu") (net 4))
 (segment (start 137.16 35.56) (end 137.16 25.4) (width 0.25) (layer "B.Cu") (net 4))
 (segment (start 148.585 45.72) (end 140.965 38.1) (width 0.25) (layer "B.Cu") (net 4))
 (segment (start 138.43 24.13) (end 144.32 24.13) (width 0.25) (layer "B.Cu") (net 4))
 (segment (start 137.16 25.4) (end 138.43 24.13) (width 0.25) (layer "B.Cu") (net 4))
 (segment (start 146.32 24.13) (end 146.32 40.915) (width 0.25) (layer "B.Cu") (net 3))
 (segment (start 144.78 50.8) (end 149.86 50.8) (width 0.25) (layer "B.Cu") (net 3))
 (segment (start 143.51 49.53) (end 144.78 50.8) (width 0.25) (layer "B.Cu") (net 3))
 (segment (start 151.13 49.53) (end 151.125 49.525) (width 0.25) (layer "B.Cu") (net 3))
 (segment (start 143.51 44.45) (end 143.51 49.53) (width 0.25) (layer "B.Cu") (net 3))
 (segment (start 146.32 40.915) (end 151.125 45.72) (width 0.25) (layer "B.Cu") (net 3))
 (segment (start 149.86 50.8) (end 151.13 49.53) (width 0.25) (layer "B.Cu") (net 3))
 (segment (start 139.7 40.64) (end 143.51 44.45) (width 0.25) (layer "B.Cu") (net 3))
 (segment (start 151.125 49.525) (end 151.125 45.72) (width 0.25) (layer "B.Cu") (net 3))
 (segment (start 139.7 43.18) (end 142.24 45.72) (width 0.25) (layer "B.Cu") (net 2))
 (segment (start 148.32 24.13) (end 148.32 40.375) (width 0.25) (layer "B.Cu") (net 2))
 (segment (start 142.24 45.72) (end 142.24 49.53) (width 0.25) (layer "B.Cu") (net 2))
 (segment (start 148.32 40.375) (end 153.665 45.72) (width 0.25) (layer "B.Cu") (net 2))
 (segment (start 149.86 52.07) (end 153.665 48.265) (width 0.25) (layer "B.Cu") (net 2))
 (segment (start 142.24 49.53) (end 144.78 52.07) (width 0.25) (layer "B.Cu") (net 2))
 (segment (start 153.665 48.265) (end 153.665 45.72) (width 0.25) (layer "B.Cu") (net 2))
 (segment (start 144.78 52.07) (end 149.86 52.07) (width 0.25) (layer "B.Cu") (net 2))
 (segment (start 139.7 48.26) (end 144.78 53.34) (width 0.25) (layer "B.Cu") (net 1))
 (segment (start 156.21 46.99) (end 156.205 46.985) (width 0.25) (layer "B.Cu") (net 1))
 (segment (start 149.86 53.34) (end 156.21 46.99) (width 0.25) (layer "B.Cu") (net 1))
 (segment (start 156.205 46.985) (end 156.205 45.72) (width 0.25) (layer "B.Cu") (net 1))
 (segment (start 156.205 33.025) (end 156.205 45.72) (width 0.25) (layer "B.Cu") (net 1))
 (segment (start 139.7 45.72) (end 139.7 48.26) (width 0.25) (layer "B.Cu") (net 1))
 (segment (start 150.32 24.13) (end 150.32 27.13) (width 0.25) (layer "B.Cu") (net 1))
 (segment (start 150.32 27.13) (end 156.21 33.02) (width 0.25) (layer "B.Cu") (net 1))
 (segment (start 144.78 53.34) (end 149.86 53.34) (width 0.25) (layer "B.Cu") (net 1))
 (segment (start 156.21 33.02) (end 156.205 33.025) (width 0.25) (layer "B.Cu") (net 1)))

